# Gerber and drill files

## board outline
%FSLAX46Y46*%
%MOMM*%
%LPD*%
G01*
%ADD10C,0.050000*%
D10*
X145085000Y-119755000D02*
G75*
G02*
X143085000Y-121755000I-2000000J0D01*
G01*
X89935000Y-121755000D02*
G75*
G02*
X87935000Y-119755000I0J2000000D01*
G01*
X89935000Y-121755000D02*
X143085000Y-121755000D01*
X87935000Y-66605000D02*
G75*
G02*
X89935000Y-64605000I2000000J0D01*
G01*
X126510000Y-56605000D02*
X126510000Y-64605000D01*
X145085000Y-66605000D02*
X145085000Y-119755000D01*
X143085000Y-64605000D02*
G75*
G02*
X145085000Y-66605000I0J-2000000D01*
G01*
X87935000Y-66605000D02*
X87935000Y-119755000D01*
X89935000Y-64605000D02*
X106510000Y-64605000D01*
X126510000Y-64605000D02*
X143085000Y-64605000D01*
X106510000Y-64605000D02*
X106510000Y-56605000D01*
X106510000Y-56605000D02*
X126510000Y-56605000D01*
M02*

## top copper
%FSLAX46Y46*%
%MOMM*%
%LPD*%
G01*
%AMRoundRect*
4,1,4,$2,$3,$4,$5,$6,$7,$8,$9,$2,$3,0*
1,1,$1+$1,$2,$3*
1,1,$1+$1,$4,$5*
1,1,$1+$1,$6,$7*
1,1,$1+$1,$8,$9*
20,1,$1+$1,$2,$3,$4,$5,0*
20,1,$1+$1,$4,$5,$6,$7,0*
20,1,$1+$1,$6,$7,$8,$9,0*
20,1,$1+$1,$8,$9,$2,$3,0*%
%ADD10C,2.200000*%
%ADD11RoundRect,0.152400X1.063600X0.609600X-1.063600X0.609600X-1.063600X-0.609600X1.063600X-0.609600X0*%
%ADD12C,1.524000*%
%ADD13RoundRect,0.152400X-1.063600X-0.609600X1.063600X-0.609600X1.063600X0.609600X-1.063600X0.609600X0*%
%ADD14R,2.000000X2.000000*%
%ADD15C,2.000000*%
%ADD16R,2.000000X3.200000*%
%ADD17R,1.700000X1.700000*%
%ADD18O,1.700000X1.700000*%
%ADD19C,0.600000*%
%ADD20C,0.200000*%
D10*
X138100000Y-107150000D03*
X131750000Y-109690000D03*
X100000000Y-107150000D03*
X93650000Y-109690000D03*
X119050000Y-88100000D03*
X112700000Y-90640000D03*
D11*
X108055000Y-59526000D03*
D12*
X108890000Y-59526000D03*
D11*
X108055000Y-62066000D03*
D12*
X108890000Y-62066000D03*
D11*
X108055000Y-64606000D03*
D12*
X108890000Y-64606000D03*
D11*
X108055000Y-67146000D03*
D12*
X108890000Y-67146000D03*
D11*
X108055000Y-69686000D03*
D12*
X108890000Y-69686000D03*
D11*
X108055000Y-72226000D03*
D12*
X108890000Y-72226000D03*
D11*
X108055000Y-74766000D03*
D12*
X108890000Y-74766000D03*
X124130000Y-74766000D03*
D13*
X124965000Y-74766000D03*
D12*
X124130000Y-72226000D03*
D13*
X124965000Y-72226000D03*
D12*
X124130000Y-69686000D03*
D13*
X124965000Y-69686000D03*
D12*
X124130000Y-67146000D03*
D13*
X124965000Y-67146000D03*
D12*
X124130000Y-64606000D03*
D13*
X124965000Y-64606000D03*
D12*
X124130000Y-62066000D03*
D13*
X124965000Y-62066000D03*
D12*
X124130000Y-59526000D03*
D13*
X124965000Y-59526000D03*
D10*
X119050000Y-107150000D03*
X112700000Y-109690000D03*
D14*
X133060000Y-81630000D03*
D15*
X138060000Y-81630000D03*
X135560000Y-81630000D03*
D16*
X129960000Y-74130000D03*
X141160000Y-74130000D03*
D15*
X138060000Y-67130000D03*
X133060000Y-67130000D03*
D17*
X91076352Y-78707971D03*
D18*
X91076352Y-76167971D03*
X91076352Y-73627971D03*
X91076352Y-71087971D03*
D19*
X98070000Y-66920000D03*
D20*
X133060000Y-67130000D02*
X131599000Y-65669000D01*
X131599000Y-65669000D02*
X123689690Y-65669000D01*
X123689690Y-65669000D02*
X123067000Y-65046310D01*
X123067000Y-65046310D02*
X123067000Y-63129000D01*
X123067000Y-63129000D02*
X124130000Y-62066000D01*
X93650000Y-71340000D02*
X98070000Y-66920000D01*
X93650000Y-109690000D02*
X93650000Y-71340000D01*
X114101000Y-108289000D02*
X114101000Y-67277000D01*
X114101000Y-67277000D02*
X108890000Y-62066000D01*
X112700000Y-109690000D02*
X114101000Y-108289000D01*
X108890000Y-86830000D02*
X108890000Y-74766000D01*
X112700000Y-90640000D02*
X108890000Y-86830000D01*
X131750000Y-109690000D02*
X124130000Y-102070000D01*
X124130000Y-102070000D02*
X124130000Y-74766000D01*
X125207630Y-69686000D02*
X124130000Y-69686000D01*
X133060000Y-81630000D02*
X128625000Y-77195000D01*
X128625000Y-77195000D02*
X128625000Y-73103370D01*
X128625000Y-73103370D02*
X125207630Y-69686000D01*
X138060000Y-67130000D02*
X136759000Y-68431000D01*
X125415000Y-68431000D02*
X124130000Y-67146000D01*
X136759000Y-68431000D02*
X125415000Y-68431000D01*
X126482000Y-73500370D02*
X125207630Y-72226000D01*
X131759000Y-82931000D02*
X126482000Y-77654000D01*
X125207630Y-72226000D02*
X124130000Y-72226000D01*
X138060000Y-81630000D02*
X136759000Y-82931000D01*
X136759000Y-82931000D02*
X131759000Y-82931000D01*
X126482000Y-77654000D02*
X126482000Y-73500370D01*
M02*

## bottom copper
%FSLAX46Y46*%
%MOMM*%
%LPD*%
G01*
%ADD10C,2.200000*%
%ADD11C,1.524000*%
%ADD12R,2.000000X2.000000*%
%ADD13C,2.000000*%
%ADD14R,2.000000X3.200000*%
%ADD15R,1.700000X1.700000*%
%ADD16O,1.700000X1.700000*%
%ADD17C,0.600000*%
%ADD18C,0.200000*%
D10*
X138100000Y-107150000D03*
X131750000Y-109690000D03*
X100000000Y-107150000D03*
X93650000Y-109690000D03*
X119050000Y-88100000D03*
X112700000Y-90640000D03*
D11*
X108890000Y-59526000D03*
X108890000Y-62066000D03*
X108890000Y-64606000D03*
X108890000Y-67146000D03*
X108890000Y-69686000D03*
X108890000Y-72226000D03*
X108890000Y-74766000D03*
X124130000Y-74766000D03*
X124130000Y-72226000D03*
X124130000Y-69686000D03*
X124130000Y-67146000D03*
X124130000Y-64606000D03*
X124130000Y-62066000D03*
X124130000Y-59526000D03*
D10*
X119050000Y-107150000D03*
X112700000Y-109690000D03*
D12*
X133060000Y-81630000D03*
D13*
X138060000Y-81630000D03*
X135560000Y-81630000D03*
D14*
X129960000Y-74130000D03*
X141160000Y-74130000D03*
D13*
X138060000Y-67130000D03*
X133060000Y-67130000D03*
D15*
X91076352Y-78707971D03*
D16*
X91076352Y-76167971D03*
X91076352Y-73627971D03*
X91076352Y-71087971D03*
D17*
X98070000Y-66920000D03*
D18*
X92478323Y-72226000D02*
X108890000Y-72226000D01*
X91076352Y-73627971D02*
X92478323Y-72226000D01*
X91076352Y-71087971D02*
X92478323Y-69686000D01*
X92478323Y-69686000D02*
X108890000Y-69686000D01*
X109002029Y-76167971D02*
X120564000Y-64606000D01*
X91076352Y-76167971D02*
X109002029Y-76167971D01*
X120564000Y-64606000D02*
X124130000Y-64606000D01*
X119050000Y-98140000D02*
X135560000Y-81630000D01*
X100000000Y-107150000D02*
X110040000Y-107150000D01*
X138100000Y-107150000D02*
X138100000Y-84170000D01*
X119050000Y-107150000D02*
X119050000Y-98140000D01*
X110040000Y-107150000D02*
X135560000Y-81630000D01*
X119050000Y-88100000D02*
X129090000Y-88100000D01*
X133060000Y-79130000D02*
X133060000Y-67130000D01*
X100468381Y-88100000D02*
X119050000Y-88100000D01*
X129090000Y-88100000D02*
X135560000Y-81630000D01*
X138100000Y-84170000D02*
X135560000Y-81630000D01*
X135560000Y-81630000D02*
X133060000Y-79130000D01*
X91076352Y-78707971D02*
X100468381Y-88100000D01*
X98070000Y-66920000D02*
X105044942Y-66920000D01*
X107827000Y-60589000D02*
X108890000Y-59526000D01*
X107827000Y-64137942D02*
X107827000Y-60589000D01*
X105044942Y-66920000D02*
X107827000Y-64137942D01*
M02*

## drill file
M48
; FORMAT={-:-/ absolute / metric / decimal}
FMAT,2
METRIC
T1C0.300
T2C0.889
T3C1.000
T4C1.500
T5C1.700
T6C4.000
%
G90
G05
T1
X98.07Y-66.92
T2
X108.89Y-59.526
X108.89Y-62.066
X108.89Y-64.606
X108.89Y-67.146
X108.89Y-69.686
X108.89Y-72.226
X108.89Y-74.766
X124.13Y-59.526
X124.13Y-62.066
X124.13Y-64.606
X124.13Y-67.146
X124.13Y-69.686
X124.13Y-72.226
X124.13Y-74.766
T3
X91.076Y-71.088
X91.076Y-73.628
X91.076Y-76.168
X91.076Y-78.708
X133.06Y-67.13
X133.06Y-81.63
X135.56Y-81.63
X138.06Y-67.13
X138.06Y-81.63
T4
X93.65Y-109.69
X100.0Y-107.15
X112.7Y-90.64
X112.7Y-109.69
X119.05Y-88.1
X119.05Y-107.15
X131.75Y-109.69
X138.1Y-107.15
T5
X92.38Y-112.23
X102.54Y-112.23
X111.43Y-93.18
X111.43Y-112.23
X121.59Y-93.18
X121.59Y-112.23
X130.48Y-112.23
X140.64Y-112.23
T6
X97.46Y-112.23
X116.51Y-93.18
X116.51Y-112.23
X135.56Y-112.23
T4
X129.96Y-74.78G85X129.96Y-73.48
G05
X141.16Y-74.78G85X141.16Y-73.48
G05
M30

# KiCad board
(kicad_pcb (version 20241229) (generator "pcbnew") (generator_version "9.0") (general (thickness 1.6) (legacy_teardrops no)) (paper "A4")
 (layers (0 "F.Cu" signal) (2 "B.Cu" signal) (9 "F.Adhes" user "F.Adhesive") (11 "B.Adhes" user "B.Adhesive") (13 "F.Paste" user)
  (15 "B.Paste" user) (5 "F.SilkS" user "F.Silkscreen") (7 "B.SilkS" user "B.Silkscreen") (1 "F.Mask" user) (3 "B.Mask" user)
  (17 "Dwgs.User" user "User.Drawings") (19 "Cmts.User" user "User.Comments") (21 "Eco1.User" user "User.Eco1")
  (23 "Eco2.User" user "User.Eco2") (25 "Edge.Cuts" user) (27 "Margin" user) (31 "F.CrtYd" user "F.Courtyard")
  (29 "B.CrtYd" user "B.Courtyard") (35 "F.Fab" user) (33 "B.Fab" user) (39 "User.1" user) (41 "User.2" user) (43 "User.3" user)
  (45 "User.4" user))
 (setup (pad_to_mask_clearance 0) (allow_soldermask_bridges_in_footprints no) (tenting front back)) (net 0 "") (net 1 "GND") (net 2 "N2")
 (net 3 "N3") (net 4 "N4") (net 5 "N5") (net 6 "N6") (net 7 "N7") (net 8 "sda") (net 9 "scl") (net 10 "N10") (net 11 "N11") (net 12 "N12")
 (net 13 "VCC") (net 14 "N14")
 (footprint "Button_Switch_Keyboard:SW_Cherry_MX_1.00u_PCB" (layer "F.Cu") (at 138.1 107.15)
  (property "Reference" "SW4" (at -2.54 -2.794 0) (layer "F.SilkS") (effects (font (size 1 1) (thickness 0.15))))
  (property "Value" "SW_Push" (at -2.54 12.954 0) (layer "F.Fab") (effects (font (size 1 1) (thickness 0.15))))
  (pad "" np_thru_hole circle (at -7.62 5.08) (size 1.7 1.7) (drill 1.7) (layers "*.Cu" "*.Mask"))
  (pad "" np_thru_hole circle (at -2.54 5.08) (size 4 4) (drill 4) (layers "*.Cu" "*.Mask"))
  (pad "" np_thru_hole circle (at 2.54 5.08) (size 1.7 1.7) (drill 1.7) (layers "*.Cu" "*.Mask"))
  (pad "1" thru_hole circle (at 0 0) (size 2.2 2.2) (drill 1.5) (layers "*.Cu" "*.Mask") (remove_unused_layers no) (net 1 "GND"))
  (pad "2" thru_hole circle (at -6.35 2.54) (size 2.2 2.2) (drill 1.5) (layers "*.Cu" "*.Mask") (remove_unused_layers no) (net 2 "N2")))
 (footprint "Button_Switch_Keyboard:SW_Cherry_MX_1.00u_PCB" (layer "F.Cu") (at 100 107.15)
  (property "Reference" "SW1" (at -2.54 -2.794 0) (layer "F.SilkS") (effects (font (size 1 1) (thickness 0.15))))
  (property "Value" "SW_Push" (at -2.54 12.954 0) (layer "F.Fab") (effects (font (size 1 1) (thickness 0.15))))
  (pad "" np_thru_hole circle (at -7.62 5.08) (size 1.7 1.7) (drill 1.7) (layers "*.Cu" "*.Mask"))
  (pad "" np_thru_hole circle (at -2.54 5.08) (size 4 4) (drill 4) (layers "*.Cu" "*.Mask"))
  (pad "" np_thru_hole circle (at 2.54 5.08) (size 1.7 1.7) (drill 1.7) (layers "*.Cu" "*.Mask"))
  (pad "1" thru_hole circle (at 0 0) (size 2.2 2.2) (drill 1.5) (layers "*.Cu" "*.Mask") (remove_unused_layers no) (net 1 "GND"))
  (pad "2" thru_hole circle (at -6.35 2.54) (size 2.2 2.2) (drill 1.5) (layers "*.Cu" "*.Mask") (remove_unused_layers no) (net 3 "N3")))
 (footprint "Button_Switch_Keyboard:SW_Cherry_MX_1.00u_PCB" (layer "F.Cu") (at 119.05 88.1)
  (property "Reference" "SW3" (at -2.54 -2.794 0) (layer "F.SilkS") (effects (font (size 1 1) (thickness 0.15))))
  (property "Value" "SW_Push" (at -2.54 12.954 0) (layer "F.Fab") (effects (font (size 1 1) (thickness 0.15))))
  (pad "" np_thru_hole circle (at -7.62 5.08) (size 1.7 1.7) (drill 1.7) (layers "*.Cu" "*.Mask"))
  (pad "" np_thru_hole circle (at -2.54 5.08) (size 4 4) (drill 4) (layers "*.Cu" "*.Mask"))
  (pad "" np_thru_hole circle (at 2.54 5.08) (size 1.7 1.7) (drill 1.7) (layers "*.Cu" "*.Mask"))
  (pad "1" thru_hole circle (at 0 0) (size 2.2 2.2) (drill 1.5) (layers "*.Cu" "*.Mask") (remove_unused_layers no) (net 1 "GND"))
  (pad "2" thru_hole circle (at -6.35 2.54) (size 2.2 2.2) (drill 1.5) (layers "*.Cu" "*.Mask") (remove_unused_layers no) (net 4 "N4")))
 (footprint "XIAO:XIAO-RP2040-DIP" (layer "F.Cu") (at 116.51 67.146)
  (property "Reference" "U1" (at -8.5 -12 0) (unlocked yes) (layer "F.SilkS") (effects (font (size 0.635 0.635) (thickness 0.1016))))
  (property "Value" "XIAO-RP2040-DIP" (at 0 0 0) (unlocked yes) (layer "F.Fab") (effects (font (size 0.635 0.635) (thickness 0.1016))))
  (pad "1" smd roundrect (at -8.455 -7.62 180) (size 2.432 1.524) (layers "F.Cu" "F.Mask") (roundrect_rratio 0.1) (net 3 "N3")
   (thermal_bridge_angle 45))
  (pad "1" thru_hole circle (at -7.62 -7.62 180) (size 1.524 1.524) (drill 0.889) (layers "*.Cu" "*.Mask") (remove_unused_layers no)
   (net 3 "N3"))
  (pad "2" smd roundrect (at -8.455 -5.08 180) (size 2.432 1.524) (layers "F.Cu" "F.Mask") (roundrect_rratio 0.1) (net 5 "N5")
   (thermal_bridge_angle 45))
  (pad "2" thru_hole circle (at -7.62 -5.08 180) (size 1.524 1.524) (drill 0.889) (layers "*.Cu" "*.Mask") (remove_unused_layers no)
   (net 5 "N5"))
  (pad "3" smd roundrect (at -8.455 -2.54 180) (size 2.432 1.524) (layers "F.Cu" "F.Mask") (roundrect_rratio 0.1) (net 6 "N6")
   (thermal_bridge_angle 45))
  (pad "3" thru_hole circle (at -7.62 -2.54 180) (size 1.524 1.524) (drill 0.889) (layers "*.Cu" "*.Mask") (remove_unused_layers no)
   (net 6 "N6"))
  (pad "4" smd roundrect (at -8.455 0 180) (size 2.432 1.524) (layers "F.Cu" "F.Mask") (roundrect_rratio 0.1) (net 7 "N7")
   (thermal_bridge_angle 45))
  (pad "4" thru_hole circle (at -7.62 0 180) (size 1.524 1.524) (drill 0.889) (layers "*.Cu" "*.Mask") (remove_unused_layers no)
   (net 7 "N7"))
  (pad "5" smd roundrect (at -8.455 2.54 180) (size 2.432 1.524) (layers "F.Cu" "F.Mask") (roundrect_rratio 0.1) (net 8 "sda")
   (thermal_bridge_angle 45))
  (pad "5" thru_hole circle (at -7.62 2.54 180) (size 1.524 1.524) (drill 0.889) (layers "*.Cu" "*.Mask") (remove_unused_layers no)
   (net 8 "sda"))
  (pad "6" smd roundrect (at -8.455 5.08 180) (size 2.432 1.524) (layers "F.Cu" "F.Mask") (roundrect_rratio 0.1) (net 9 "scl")
   (thermal_bridge_angle 45))
  (pad "6" thru_hole circle (at -7.62 5.08 180) (size 1.524 1.524) (drill 0.889) (layers "*.Cu" "*.Mask") (remove_unused_layers no)
   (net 9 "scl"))
  (pad "7" smd roundrect (at -8.455 7.62 180) (size 2.432 1.524) (layers "F.Cu" "F.Mask") (roundrect_rratio 0.1) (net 4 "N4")
   (thermal_bridge_angle 45))
  (pad "7" thru_hole circle (at -7.62 7.62 180) (size 1.524 1.524) (drill 0.889) (layers "*.Cu" "*.Mask") (remove_unused_layers no)
   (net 4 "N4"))
  (pad "8" thru_hole circle (at 7.62 7.62) (size 1.524 1.524) (drill 0.889) (layers "*.Cu" "*.Mask") (remove_unused_layers no) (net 2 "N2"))
  (pad "8" smd roundrect (at 8.455 7.62) (size 2.432 1.524) (layers "F.Cu" "F.Mask") (roundrect_rratio 0.1) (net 2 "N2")
   (thermal_bridge_angle 45))
  (pad "9" thru_hole circle (at 7.62 5.08) (size 1.524 1.524) (drill 0.889) (layers "*.Cu" "*.Mask") (remove_unused_layers no)
   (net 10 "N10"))
  (pad "9" smd roundrect (at 8.455 5.08) (size 2.432 1.524) (layers "F.Cu" "F.Mask") (roundrect_rratio 0.1) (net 10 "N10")
   (thermal_bridge_angle 45))
  (pad "10" thru_hole circle (at 7.62 2.54) (size 1.524 1.524) (drill 0.889) (layers "*.Cu" "*.Mask") (remove_unused_layers no)
   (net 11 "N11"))
  (pad "10" smd roundrect (at 8.455 2.54) (size 2.432 1.524) (layers "F.Cu" "F.Mask") (roundrect_rratio 0.1) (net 11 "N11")
   (thermal_bridge_angle 45))
  (pad "11" thru_hole circle (at 7.62 0) (size 1.524 1.524) (drill 0.889) (layers "*.Cu" "*.Mask") (remove_unused_layers no) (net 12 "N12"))
  (pad "11" smd roundrect (at 8.455 0) (size 2.432 1.524) (layers "F.Cu" "F.Mask") (roundrect_rratio 0.1) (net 12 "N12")
   (thermal_bridge_angle 45))
  (pad "12" thru_hole circle (at 7.62 -2.54) (size 1.524 1.524) (drill 0.889) (layers "*.Cu" "*.Mask") (remove_unused_layers no)
   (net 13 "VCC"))
  (pad "12" smd roundrect (at 8.455 -2.54) (size 2.432 1.524) (layers "F.Cu" "F.Mask") (roundrect_rratio 0.1) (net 13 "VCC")
   (thermal_bridge_angle 45))
  (pad "13" thru_hole circle (at 7.62 -5.08) (size 1.524 1.524) (drill 0.889) (layers "*.Cu" "*.Mask") (remove_unused_layers no)
   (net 1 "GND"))
  (pad "13" smd roundrect (at 8.455 -5.08) (size 2.432 1.524) (layers "F.Cu" "F.Mask") (roundrect_rratio 0.1) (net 1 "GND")
   (thermal_bridge_angle 45))
  (pad "14" thru_hole circle (at 7.62 -7.62) (size 1.524 1.524) (drill 0.889) (layers "*.Cu" "*.Mask") (remove_unused_layers no)
   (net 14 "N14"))
  (pad "14" smd roundrect (at 8.455 -7.62) (size 2.432 1.524) (layers "F.Cu" "F.Mask") (roundrect_rratio 0.1) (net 14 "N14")
   (thermal_bridge_angle 45)))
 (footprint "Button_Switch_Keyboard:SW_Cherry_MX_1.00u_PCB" (layer "F.Cu") (at 119.05 107.15)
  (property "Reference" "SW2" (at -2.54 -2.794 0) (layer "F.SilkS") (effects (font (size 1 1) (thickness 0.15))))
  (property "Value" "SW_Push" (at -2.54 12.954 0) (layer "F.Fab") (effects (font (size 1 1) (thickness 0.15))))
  (pad "" np_thru_hole circle (at -7.62 5.08) (size 1.7 1.7) (drill 1.7) (layers "*.Cu" "*.Mask"))
  (pad "" np_thru_hole circle (at -2.54 5.08) (size 4 4) (drill 4) (layers "*.Cu" "*.Mask"))
  (pad "" np_thru_hole circle (at 2.54 5.08) (size 1.7 1.7) (drill 1.7) (layers "*.Cu" "*.Mask"))
  (pad "1" thru_hole circle (at 0 0) (size 2.2 2.2) (drill 1.5) (layers "*.Cu" "*.Mask") (remove_unused_layers no) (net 1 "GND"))
  (pad "2" thru_hole circle (at -6.35 2.54) (size 2.2 2.2) (drill 1.5) (layers "*.Cu" "*.Mask") (remove_unused_layers no) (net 5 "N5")))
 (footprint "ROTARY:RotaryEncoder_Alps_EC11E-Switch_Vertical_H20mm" (layer "F.Cu") (at 133.06 81.63 90)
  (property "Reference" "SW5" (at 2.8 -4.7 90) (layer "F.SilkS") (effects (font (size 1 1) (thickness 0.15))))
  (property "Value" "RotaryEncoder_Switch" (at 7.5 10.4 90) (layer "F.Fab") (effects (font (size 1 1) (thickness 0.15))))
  (pad "A" thru_hole rect (at 0 0 90) (size 2 2) (drill 1) (layers "*.Cu" "*.Mask") (remove_unused_layers no) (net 11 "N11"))
  (pad "B" thru_hole circle (at 0 5 90) (size 2 2) (drill 1) (layers "*.Cu" "*.Mask") (remove_unused_layers no) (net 10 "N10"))
  (pad "C" thru_hole circle (at 0 2.5 90) (size 2 2) (drill 1) (layers "*.Cu" "*.Mask") (remove_unused_layers no) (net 1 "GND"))
  (pad "MP" thru_hole rect (at 7.5 -3.1 90) (size 3.2 2) (drill oval 2.8 1.5) (layers "*.Cu" "*.Mask") (remove_unused_layers no))
  (pad "MP" thru_hole rect (at 7.5 8.1 90) (size 3.2 2) (drill oval 2.8 1.5) (layers "*.Cu" "*.Mask") (remove_unused_layers no))
  (pad "S1" thru_hole circle (at 14.5 5 90) (size 2 2) (drill 1) (layers "*.Cu" "*.Mask") (remove_unused_layers no) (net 12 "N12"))
  (pad "S2" thru_hole circle (at 14.5 0 90) (size 2 2) (drill 1) (layers "*.Cu" "*.Mask") (remove_unused_layers no) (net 1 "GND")))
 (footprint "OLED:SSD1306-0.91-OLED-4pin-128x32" (layer "F.Cu") (at 127.576352 80.897971 180)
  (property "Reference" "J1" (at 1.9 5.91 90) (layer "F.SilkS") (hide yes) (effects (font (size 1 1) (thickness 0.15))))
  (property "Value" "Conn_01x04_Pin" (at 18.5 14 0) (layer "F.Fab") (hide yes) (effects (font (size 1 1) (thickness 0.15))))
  (pad "1" thru_hole rect (at 36.5 2.19 180) (size 1.7 1.7) (drill 1) (layers "*.Cu" "*.Mask") (remove_unused_layers no) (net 1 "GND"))
  (pad "2" thru_hole oval (at 36.5 4.73 180) (size 1.7 1.7) (drill 1) (layers "*.Cu" "*.Mask") (remove_unused_layers no) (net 13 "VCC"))
  (pad "3" thru_hole oval (at 36.5 7.27 180) (size 1.7 1.7) (drill 1) (layers "*.Cu" "*.Mask") (remove_unused_layers no) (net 9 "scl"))
  (pad "4" thru_hole oval (at 36.5 9.81 180) (size 1.7 1.7) (drill 1) (layers "*.Cu" "*.Mask") (remove_unused_layers no) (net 8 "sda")))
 (gr_arc (start 145.085 119.755) (mid 144.499214 121.169214) (end 143.085 121.755) (stroke (width 0.05) (type default)) (layer "Edge.Cuts"))
 (gr_arc (start 89.935 121.755) (mid 88.520786 121.169214) (end 87.935 119.755) (stroke (width 0.05) (type default)) (layer "Edge.Cuts"))
 (gr_line (start 89.935 121.755) (end 143.085 121.755) (stroke (width 0.05) (type solid)) (layer "Edge.Cuts"))
 (gr_arc (start 87.935 66.605) (mid 88.520786 65.190786) (end 89.935 64.605) (stroke (width 0.05) (type default)) (layer "Edge.Cuts"))
 (gr_line (start 126.51 56.605) (end 126.51 64.605) (stroke (width 0.05) (type solid)) (layer "Edge.Cuts"))
 (gr_line (start 145.085 66.605) (end 145.085 119.755) (stroke (width 0.05) (type solid)) (layer "Edge.Cuts"))
 (gr_arc (start 143.085 64.605) (mid 144.499214 65.190786) (end 145.085 66.605) (stroke (width 0.05) (type default)) (layer "Edge.Cuts"))
 (gr_line (start 87.935 66.605) (end 87.935 119.755) (stroke (width 0.05) (type solid)) (layer "Edge.Cuts"))
 (gr_line (start 89.935 64.605) (end 106.51 64.605) (stroke (width 0.05) (type solid)) (layer "Edge.Cuts"))
 (gr_line (start 126.51 64.605) (end 143.085 64.605) (stroke (width 0.05) (type solid)) (layer "Edge.Cuts"))
 (gr_line (start 106.51 64.605) (end 106.51 56.605) (stroke (width 0.05) (type solid)) (layer "Edge.Cuts"))
 (gr_line (start 106.51 56.605) (end 126.51 56.605) (stroke (width 0.05) (type solid)) (layer "Edge.Cuts"))
 (segment (start 92.478323 72.226) (end 108.89 72.226) (width 0.2) (layer "B.Cu") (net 9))
 (segment (start 91.076352 73.627971) (end 92.478323 72.226) (width 0.2) (layer "B.Cu") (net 9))
 (segment (start 91.076352 71.087971) (end 92.478323 69.686) (width 0.2) (layer "B.Cu") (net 8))
 (segment (start 92.478323 69.686) (end 108.89 69.686) (width 0.2) (layer "B.Cu") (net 8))
 (segment (start 109.002029 76.167971) (end 120.564 64.606) (width 0.2) (layer "B.Cu") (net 13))
 (segment (start 91.076352 76.167971) (end 109.002029 76.167971) (width 0.2) (layer "B.Cu") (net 13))
 (segment (start 120.564 64.606) (end 124.13 64.606) (width 0.2) (layer "B.Cu") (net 13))
 (segment (start 133.06 67.13) (end 131.599 65.669) (width 0.2) (layer "F.Cu") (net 1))
 (segment (start 131.599 65.669) (end 123.68969 65.669) (width 0.2) (layer "F.Cu") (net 1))
 (segment (start 123.68969 65.669) (end 123.067 65.04631) (width 0.2) (layer "F.Cu") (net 1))
 (segment (start 123.067 65.04631) (end 123.067 63.129) (width 0.2) (layer "F.Cu") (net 1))
 (segment (start 123.067 63.129) (end 124.13 62.066) (width 0.2) (layer "F.Cu") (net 1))
 (segment (start 119.05 98.14) (end 135.56 81.63) (width 0.2) (layer "B.Cu") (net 1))
 (segment (start 100 107.15) (end 110.04 107.15) (width 0.2) (layer "B.Cu") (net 1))
 (segment (start 138.1 107.15) (end 138.1 84.17) (width 0.2) (layer "B.Cu") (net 1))
 (segment (start 119.05 107.15) (end 119.05 98.14) (width 0.2) (layer "B.Cu") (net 1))
 (segment (start 110.04 107.15) (end 135.56 81.63) (width 0.2) (layer "B.Cu") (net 1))
 (segment (start 119.05 88.1) (end 129.09 88.1) (width 0.2) (layer "B.Cu") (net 1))
 (segment (start 133.06 79.13) (end 133.06 67.13) (width 0.2) (layer "B.Cu") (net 1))
 (segment (start 100.468381 88.1) (end 119.05 88.1) (width 0.2) (layer "B.Cu") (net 1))
 (segment (start 129.09 88.1) (end 135.56 81.63) (width 0.2) (layer "B.Cu") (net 1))
 (segment (start 138.1 84.17) (end 135.56 81.63) (width 0.2) (layer "B.Cu") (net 1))
 (segment (start 135.56 81.63) (end 133.06 79.13) (width 0.2) (layer "B.Cu") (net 1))
 (segment (start 91.076352 78.707971) (end 100.468381 88.1) (width 0.2) (layer "B.Cu") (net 1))
 (segment (start 93.65 71.34) (end 98.07 66.92) (width 0.2) (layer "F.Cu") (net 3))
 (segment (start 93.65 109.69) (end 93.65 71.34) (width 0.2) (layer "F.Cu") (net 3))
 (via (at 98.07 66.92) (size 0.6) (drill 0.3) (layers "F.Cu" "B.Cu") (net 3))
 (segment (start 98.07 66.92) (end 105.044942 66.92) (width 0.2) (layer "B.Cu") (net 3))
 (segment (start 107.827 60.589) (end 108.89 59.526) (width 0.2) (layer "B.Cu") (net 3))
 (segment (start 107.827 64.137942) (end 107.827 60.589) (width 0.2) (layer "B.Cu") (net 3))
 (segment (start 105.044942 66.92) (end 107.827 64.137942) (width 0.2) (layer "B.Cu") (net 3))
 (segment (start 114.101 108.289) (end 114.101 67.277) (width 0.2) (layer "F.Cu") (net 5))
 (segment (start 114.101 67.277) (end 108.89 62.066) (width 0.2) (layer "F.Cu") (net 5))
 (segment (start 112.7 109.69) (end 114.101 108.289) (width 0.2) (layer "F.Cu") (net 5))
 (segment (start 108.89 86.83) (end 108.89 74.766) (width 0.2) (layer "F.Cu") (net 4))
 (segment (start 112.7 90.64) (end 108.89 86.83) (width 0.2) (layer "F.Cu") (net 4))
 (segment (start 131.75 109.69) (end 124.13 102.07) (width 0.2) (layer "F.Cu") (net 2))
 (segment (start 124.13 102.07) (end 124.13 74.766) (width 0.2) (layer "F.Cu") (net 2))
 (segment (start 125.20763 69.686) (end 124.13 69.686) (width 0.2) (layer "F.Cu") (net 11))
 (segment (start 133.06 81.63) (end 128.625 77.195) (width 0.2) (layer "F.Cu") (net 11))
 (segment (start 128.625 77.195) (end 128.625 73.10337) (width 0.2) (layer "F.Cu") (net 11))
 (segment (start 128.625 73.10337) (end 125.20763 69.686) (width 0.2) (layer "F.Cu") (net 11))
 (segment (start 138.06 67.13) (end 136.759 68.431) (width 0.2) (layer "F.Cu") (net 12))
 (segment (start 125.415 68.431) (end 124.13 67.146) (width 0.2) (layer "F.Cu") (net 12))
 (segment (start 136.759 68.431) (end 125.415 68.431) (width 0.2) (layer "F.Cu") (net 12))
 (segment (start 126.482 73.50037) (end 125.20763 72.226) (width 0.2) (layer "F.Cu") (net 10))
 (segment (start 131.759 82.931) (end 126.482 77.654) (width 0.2) (layer "F.Cu") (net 10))
 (segment (start 125.20763 72.226) (end 124.13 72.226) (width 0.2) (layer "F.Cu") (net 10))
 (segment (start 138.06 81.63) (end 136.759 82.931) (width 0.2) (layer "F.Cu") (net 10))
 (segment (start 136.759 82.931) (end 131.759 82.931) (width 0.2) (layer "F.Cu") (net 10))
 (segment (start 126.482 77.654) (end 126.482 73.50037) (width 0.2) (layer "F.Cu") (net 10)))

